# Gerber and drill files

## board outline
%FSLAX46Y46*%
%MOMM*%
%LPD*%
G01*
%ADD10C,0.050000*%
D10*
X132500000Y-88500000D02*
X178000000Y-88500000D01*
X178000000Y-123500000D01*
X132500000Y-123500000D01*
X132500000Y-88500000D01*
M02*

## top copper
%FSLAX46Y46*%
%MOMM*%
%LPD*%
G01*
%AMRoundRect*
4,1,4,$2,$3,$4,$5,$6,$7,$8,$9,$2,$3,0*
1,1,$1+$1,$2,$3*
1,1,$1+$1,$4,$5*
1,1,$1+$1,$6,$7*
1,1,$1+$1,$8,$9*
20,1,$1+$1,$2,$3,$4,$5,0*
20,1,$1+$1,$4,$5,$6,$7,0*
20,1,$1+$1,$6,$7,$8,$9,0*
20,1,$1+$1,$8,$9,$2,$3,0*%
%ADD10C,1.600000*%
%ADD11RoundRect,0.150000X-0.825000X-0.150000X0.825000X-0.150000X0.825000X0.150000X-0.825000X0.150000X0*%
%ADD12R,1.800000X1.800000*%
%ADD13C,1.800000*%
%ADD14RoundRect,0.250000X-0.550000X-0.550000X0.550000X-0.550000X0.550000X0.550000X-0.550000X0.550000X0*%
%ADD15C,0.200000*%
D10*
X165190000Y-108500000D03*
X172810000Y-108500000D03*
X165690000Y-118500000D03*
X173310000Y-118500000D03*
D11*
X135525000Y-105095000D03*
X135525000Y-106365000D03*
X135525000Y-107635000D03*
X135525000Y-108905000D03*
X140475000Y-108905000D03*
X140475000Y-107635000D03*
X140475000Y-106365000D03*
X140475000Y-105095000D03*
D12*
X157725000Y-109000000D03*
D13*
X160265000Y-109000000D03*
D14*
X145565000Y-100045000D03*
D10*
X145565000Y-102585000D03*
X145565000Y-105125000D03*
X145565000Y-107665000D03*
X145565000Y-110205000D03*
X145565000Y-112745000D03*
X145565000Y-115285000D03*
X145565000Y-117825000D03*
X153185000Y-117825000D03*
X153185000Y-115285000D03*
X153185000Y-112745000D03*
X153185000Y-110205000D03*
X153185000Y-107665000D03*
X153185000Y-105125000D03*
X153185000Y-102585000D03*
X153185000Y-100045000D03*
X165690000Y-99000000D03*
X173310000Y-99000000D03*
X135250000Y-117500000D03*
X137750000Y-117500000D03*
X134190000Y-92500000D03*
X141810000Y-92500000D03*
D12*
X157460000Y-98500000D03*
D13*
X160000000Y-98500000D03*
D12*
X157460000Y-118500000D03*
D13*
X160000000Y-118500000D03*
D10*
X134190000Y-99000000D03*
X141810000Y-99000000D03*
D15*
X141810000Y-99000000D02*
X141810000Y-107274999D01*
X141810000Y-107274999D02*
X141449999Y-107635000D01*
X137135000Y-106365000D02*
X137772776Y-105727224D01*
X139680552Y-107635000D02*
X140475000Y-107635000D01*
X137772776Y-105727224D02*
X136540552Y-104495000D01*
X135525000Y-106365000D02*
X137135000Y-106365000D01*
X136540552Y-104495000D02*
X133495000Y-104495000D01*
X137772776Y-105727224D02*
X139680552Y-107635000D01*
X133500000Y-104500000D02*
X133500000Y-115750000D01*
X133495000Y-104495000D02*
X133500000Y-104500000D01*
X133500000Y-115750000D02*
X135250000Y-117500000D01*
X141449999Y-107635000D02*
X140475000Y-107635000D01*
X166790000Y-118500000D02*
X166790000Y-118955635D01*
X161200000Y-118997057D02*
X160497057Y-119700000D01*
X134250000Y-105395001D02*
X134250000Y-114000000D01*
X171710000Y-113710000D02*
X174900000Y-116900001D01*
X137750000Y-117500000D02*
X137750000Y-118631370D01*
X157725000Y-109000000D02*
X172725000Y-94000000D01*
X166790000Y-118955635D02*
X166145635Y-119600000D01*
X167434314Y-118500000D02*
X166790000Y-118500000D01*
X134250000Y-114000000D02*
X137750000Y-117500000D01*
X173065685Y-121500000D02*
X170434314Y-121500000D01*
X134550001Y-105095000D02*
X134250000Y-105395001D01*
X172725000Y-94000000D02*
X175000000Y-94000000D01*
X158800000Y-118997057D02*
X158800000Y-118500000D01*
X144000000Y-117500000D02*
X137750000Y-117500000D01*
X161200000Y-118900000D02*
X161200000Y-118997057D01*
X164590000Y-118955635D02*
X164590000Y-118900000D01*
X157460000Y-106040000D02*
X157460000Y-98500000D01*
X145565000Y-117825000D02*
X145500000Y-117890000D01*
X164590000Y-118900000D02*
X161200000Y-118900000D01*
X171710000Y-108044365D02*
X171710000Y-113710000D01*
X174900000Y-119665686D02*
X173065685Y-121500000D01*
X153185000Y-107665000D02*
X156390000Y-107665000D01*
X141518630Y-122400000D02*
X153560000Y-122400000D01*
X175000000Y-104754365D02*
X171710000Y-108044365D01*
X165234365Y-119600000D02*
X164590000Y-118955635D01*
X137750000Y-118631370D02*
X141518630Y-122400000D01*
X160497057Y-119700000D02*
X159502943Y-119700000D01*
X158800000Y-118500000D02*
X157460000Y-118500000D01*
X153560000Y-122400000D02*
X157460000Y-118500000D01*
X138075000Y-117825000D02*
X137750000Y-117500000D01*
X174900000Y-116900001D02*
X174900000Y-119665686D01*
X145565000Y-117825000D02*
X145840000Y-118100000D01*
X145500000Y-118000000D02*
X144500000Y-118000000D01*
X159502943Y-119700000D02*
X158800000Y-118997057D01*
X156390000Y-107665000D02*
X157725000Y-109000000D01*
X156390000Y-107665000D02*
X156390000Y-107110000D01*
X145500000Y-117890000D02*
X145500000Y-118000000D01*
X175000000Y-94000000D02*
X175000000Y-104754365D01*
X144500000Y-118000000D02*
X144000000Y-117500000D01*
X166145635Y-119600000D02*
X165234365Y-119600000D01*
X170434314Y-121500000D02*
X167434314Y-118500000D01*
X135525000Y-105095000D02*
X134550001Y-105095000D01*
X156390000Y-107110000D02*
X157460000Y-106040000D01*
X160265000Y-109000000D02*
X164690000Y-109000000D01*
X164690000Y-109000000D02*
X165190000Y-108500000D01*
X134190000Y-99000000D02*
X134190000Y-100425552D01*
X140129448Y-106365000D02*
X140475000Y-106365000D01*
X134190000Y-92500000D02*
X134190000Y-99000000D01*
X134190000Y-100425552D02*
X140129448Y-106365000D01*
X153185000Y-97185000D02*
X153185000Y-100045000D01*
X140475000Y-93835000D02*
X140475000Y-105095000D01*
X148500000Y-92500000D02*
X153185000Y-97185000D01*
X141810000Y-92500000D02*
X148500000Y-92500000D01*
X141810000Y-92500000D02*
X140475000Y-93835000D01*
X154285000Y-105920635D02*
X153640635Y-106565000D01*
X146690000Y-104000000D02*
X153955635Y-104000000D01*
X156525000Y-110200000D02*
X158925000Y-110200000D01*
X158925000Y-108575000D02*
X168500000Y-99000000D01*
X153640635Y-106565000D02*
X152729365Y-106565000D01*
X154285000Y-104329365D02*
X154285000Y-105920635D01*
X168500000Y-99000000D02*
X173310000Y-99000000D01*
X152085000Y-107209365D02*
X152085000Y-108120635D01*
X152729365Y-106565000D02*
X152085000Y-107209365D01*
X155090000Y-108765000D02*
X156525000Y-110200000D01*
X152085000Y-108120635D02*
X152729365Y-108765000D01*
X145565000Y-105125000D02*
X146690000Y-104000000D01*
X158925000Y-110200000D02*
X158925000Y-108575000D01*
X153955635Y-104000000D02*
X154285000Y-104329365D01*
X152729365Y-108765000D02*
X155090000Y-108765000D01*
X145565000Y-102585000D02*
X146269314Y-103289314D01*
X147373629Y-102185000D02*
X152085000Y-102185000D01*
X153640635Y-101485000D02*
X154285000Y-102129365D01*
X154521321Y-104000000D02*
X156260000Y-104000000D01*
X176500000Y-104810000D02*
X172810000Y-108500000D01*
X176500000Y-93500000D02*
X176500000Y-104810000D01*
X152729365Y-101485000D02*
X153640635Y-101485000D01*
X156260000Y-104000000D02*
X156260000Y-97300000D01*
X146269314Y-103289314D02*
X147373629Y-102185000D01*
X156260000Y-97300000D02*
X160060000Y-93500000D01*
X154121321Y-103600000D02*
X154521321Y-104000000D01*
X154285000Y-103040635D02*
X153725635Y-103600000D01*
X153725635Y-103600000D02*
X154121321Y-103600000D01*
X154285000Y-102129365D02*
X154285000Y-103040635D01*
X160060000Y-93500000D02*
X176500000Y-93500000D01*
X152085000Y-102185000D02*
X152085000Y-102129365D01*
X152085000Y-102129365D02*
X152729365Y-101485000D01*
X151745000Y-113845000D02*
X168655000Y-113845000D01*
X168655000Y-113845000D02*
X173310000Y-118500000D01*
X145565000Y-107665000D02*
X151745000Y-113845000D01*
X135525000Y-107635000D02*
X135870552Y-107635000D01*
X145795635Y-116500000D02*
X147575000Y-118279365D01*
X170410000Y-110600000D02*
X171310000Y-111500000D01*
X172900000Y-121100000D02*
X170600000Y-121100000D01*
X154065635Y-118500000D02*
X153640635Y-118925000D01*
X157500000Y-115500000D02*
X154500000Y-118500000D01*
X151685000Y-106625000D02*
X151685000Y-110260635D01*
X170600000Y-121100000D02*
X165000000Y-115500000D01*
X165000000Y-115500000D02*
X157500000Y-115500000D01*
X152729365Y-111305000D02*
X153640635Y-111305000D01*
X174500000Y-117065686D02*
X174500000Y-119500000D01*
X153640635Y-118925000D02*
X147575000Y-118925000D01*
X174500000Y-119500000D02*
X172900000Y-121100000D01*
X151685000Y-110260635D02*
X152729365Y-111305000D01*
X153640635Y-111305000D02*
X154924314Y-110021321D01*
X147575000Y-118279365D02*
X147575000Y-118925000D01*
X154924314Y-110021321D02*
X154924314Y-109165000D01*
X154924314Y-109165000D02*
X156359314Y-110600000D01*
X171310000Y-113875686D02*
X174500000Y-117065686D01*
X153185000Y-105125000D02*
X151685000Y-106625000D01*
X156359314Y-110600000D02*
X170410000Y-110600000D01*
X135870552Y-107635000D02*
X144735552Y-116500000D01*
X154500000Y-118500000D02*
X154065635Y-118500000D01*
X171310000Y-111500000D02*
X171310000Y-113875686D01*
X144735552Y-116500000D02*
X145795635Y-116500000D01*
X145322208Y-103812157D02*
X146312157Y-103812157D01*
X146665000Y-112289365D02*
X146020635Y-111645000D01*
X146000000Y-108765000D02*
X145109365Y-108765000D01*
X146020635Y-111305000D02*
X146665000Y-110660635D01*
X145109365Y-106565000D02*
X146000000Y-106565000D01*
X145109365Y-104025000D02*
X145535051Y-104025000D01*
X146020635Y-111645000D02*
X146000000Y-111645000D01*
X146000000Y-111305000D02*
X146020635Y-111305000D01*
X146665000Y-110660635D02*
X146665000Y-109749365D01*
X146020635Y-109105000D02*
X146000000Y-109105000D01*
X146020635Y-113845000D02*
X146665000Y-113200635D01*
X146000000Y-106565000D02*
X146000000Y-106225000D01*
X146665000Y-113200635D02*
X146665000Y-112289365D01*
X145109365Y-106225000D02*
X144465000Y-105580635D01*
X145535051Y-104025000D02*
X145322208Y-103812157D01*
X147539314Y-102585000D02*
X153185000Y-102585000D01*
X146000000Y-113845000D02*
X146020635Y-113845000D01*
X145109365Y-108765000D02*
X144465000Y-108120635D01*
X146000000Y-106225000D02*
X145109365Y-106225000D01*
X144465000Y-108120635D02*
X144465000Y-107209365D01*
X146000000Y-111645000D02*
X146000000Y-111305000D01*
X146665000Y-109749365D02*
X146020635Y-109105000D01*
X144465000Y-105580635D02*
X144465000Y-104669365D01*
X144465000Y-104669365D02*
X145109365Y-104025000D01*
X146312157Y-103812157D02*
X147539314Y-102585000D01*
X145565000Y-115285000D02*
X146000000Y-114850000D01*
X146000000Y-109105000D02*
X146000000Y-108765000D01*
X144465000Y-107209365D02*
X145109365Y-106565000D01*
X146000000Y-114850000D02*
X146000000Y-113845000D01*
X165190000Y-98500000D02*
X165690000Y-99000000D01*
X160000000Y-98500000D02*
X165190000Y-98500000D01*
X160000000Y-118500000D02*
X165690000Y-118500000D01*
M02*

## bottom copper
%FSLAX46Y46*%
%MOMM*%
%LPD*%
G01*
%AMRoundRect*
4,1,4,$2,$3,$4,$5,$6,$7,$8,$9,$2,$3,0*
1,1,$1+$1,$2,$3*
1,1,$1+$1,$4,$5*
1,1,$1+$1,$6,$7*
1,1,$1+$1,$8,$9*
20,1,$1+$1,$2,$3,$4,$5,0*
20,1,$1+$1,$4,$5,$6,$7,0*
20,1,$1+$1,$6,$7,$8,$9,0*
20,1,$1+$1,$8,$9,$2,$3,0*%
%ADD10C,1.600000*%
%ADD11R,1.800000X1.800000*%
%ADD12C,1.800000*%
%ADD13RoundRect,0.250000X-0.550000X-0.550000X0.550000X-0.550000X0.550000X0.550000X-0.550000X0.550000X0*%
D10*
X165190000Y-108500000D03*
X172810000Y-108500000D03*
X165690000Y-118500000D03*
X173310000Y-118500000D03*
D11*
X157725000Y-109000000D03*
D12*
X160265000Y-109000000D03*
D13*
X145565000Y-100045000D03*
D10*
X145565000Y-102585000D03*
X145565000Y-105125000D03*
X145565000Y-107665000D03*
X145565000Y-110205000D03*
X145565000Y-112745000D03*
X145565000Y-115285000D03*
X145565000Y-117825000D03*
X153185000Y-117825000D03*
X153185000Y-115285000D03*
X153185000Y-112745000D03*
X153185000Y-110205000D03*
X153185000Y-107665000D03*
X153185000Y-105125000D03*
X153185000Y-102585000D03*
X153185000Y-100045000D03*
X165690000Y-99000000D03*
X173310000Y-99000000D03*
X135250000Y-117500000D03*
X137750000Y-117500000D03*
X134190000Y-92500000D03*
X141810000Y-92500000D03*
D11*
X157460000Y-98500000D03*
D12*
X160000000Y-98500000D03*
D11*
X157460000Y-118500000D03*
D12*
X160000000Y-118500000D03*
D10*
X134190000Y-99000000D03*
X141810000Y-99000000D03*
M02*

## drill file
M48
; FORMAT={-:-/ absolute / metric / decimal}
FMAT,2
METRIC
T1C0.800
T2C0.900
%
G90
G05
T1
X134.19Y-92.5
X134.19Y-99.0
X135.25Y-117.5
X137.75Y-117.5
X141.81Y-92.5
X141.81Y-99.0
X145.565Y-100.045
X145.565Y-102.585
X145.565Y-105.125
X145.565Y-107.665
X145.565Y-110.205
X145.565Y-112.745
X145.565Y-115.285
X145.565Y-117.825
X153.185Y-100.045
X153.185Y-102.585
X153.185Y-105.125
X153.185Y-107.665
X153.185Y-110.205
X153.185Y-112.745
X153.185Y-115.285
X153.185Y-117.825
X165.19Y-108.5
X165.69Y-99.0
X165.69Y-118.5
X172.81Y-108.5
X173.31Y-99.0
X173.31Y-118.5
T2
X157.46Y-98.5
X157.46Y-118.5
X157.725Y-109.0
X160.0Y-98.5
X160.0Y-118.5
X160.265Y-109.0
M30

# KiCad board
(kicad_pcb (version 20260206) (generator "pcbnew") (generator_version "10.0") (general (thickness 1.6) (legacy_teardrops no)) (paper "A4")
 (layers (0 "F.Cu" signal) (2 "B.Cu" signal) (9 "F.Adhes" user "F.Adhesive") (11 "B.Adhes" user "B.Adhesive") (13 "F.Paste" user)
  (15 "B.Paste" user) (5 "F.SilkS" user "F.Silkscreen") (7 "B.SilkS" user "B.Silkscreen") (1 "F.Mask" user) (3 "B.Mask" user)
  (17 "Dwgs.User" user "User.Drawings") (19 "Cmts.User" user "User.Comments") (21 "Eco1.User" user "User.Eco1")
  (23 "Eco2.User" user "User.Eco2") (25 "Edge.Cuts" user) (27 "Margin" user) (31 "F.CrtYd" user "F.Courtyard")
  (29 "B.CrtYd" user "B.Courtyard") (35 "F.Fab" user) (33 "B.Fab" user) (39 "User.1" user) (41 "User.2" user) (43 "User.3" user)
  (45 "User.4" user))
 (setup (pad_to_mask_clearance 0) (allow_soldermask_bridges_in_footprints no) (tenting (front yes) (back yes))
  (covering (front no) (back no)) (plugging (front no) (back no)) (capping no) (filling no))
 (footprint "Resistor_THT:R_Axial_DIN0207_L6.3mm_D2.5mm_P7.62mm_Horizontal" (layer "F.Cu") (at 165.19 108.5)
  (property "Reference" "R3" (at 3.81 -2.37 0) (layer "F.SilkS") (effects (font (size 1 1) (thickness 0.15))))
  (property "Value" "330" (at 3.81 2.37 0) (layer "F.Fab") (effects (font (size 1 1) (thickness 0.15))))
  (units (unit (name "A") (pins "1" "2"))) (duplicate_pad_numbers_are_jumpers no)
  (pad "1" thru_hole circle (at 0 0) (size 1.6 1.6) (drill 0.8) (layers "*.Cu" "*.Mask") (remove_unused_layers no) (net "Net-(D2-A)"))
  (pad "2" thru_hole circle (at 7.62 0) (size 1.6 1.6) (drill 0.8) (layers "*.Cu" "*.Mask") (remove_unused_layers no) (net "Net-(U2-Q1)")))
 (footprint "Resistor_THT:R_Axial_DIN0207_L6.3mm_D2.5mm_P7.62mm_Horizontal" (layer "F.Cu") (at 165.69 118.5)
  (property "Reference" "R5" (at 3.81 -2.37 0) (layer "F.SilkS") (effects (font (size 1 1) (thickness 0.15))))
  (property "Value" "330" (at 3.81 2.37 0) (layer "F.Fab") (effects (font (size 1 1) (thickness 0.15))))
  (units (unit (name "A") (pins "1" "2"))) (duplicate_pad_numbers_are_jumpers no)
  (pad "1" thru_hole circle (at 0 0) (size 1.6 1.6) (drill 0.8) (layers "*.Cu" "*.Mask") (remove_unused_layers no) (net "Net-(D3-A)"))
  (pad "2" thru_hole circle (at 7.62 0) (size 1.6 1.6) (drill 0.8) (layers "*.Cu" "*.Mask") (remove_unused_layers no) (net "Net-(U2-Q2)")))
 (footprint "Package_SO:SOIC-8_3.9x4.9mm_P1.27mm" (layer "F.Cu") (at 138 107)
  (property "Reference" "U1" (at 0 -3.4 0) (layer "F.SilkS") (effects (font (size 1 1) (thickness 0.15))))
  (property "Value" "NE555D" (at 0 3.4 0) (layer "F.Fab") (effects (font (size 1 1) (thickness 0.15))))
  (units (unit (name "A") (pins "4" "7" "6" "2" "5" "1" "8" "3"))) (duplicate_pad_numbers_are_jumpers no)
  (pad "1" smd roundrect (at -2.475 -1.905) (size 1.95 0.6) (layers "F.Cu" "F.Mask" "F.Paste") (roundrect_rratio 0.25) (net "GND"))
  (pad "2" smd roundrect (at -2.475 -0.635) (size 1.95 0.6) (layers "F.Cu" "F.Mask" "F.Paste") (roundrect_rratio 0.25)
   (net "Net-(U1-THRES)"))
  (pad "3" smd roundrect (at -2.475 0.635) (size 1.95 0.6) (layers "F.Cu" "F.Mask" "F.Paste") (roundrect_rratio 0.25) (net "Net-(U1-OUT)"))
  (pad "4" smd roundrect (at -2.475 1.905) (size 1.95 0.6) (layers "F.Cu" "F.Mask" "F.Paste") (roundrect_rratio 0.25)
   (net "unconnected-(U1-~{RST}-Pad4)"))
  (pad "5" smd roundrect (at 2.475 1.905) (size 1.95 0.6) (layers "F.Cu" "F.Mask" "F.Paste") (roundrect_rratio 0.25)
   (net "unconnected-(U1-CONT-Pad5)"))
  (pad "6" smd roundrect (at 2.475 0.635) (size 1.95 0.6) (layers "F.Cu" "F.Mask" "F.Paste") (roundrect_rratio 0.25) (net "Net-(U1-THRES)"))
  (pad "7" smd roundrect (at 2.475 -0.635) (size 1.95 0.6) (layers "F.Cu" "F.Mask" "F.Paste") (roundrect_rratio 0.25) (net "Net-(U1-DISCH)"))
  (pad "8" smd roundrect (at 2.475 -1.905) (size 1.95 0.6) (layers "F.Cu" "F.Mask" "F.Paste") (roundrect_rratio 0.25) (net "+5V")))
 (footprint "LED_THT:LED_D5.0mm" (layer "F.Cu") (at 157.725 109)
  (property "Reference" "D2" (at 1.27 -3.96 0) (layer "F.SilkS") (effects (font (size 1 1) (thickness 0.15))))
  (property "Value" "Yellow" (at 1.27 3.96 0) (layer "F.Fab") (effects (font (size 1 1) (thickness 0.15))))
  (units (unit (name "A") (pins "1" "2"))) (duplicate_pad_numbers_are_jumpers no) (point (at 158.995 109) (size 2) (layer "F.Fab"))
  (pad "1" thru_hole rect (at 0 0) (size 1.8 1.8) (drill 0.9) (layers "*.Cu" "*.Mask") (remove_unused_layers no) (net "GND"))
  (pad "2" thru_hole circle (at 2.54 0) (size 1.8 1.8) (drill 0.9) (layers "*.Cu" "*.Mask") (remove_unused_layers no) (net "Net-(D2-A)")))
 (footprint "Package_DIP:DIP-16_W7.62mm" (layer "F.Cu") (at 145.565 100.045)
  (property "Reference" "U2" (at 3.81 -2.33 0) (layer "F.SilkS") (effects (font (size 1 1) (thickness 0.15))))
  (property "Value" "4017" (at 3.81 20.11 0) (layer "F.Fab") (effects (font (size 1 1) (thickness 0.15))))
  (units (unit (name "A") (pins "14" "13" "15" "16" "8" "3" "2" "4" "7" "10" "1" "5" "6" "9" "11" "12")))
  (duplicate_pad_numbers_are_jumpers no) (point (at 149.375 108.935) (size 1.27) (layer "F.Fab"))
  (pad "1" thru_hole roundrect (at 0 0) (size 1.6 1.6) (drill 0.8) (layers "*.Cu" "*.Mask") (remove_unused_layers no)
   (roundrect_rratio 0.15625) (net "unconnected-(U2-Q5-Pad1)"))
  (pad "2" thru_hole circle (at 0 2.54) (size 1.6 1.6) (drill 0.8) (layers "*.Cu" "*.Mask") (remove_unused_layers no) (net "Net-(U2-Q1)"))
  (pad "3" thru_hole circle (at 0 5.08) (size 1.6 1.6) (drill 0.8) (layers "*.Cu" "*.Mask") (remove_unused_layers no) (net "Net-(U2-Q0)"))
  (pad "4" thru_hole circle (at 0 7.62) (size 1.6 1.6) (drill 0.8) (layers "*.Cu" "*.Mask") (remove_unused_layers no) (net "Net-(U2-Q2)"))
  (pad "5" thru_hole circle (at 0 10.16) (size 1.6 1.6) (drill 0.8) (layers "*.Cu" "*.Mask") (remove_unused_layers no)
   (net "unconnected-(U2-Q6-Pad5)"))
  (pad "6" thru_hole circle (at 0 12.7) (size 1.6 1.6) (drill 0.8) (layers "*.Cu" "*.Mask") (remove_unused_layers no)
   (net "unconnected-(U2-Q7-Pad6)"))
  (pad "7" thru_hole circle (at 0 15.24) (size 1.6 1.6) (drill 0.8) (layers "*.Cu" "*.Mask") (remove_unused_layers no) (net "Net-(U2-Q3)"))
  (pad "8" thru_hole circle (at 0 17.78) (size 1.6 1.6) (drill 0.8) (layers "*.Cu" "*.Mask") (remove_unused_layers no) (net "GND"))
  (pad "9" thru_hole circle (at 7.62 17.78) (size 1.6 1.6) (drill 0.8) (layers "*.Cu" "*.Mask") (remove_unused_layers no)
   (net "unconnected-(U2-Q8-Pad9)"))
  (pad "10" thru_hole circle (at 7.62 15.24) (size 1.6 1.6) (drill 0.8) (layers "*.Cu" "*.Mask") (remove_unused_layers no)
   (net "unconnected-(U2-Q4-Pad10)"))
  (pad "11" thru_hole circle (at 7.62 12.7) (size 1.6 1.6) (drill 0.8) (layers "*.Cu" "*.Mask") (remove_unused_layers no)
   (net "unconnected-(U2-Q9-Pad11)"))
  (pad "12" thru_hole circle (at 7.62 10.16) (size 1.6 1.6) (drill 0.8) (layers "*.Cu" "*.Mask") (remove_unused_layers no)
   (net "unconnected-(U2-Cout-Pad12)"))
  (pad "13" thru_hole circle (at 7.62 7.62) (size 1.6 1.6) (drill 0.8) (layers "*.Cu" "*.Mask") (remove_unused_layers no) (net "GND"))
  (pad "14" thru_hole circle (at 7.62 5.08) (size 1.6 1.6) (drill 0.8) (layers "*.Cu" "*.Mask") (remove_unused_layers no)
   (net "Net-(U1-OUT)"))
  (pad "15" thru_hole circle (at 7.62 2.54) (size 1.6 1.6) (drill 0.8) (layers "*.Cu" "*.Mask") (remove_unused_layers no)
   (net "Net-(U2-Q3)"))
  (pad "16" thru_hole circle (at 7.62 0) (size 1.6 1.6) (drill 0.8) (layers "*.Cu" "*.Mask") (remove_unused_layers no) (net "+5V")))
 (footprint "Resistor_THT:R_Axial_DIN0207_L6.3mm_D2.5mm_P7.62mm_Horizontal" (layer "F.Cu") (at 165.69 99)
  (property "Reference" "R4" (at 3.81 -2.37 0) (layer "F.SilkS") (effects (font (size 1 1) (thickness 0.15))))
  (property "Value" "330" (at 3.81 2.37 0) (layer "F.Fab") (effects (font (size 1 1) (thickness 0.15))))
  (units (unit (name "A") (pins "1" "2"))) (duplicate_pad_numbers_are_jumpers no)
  (pad "1" thru_hole circle (at 0 0) (size 1.6 1.6) (drill 0.8) (layers "*.Cu" "*.Mask") (remove_unused_layers no) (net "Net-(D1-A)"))
  (pad "2" thru_hole circle (at 7.62 0) (size 1.6 1.6) (drill 0.8) (layers "*.Cu" "*.Mask") (remove_unused_layers no) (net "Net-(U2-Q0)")))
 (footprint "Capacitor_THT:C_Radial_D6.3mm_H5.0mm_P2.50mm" (layer "F.Cu") (at 135.25 117.5)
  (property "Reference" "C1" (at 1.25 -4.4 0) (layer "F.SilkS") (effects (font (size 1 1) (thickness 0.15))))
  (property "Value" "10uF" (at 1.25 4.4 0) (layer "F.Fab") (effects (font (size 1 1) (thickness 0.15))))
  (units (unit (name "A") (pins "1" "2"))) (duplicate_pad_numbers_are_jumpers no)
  (pad "1" thru_hole circle (at 0 0) (size 1.6 1.6) (drill 0.8) (layers "*.Cu" "*.Mask") (remove_unused_layers no) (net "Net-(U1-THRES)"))
  (pad "2" thru_hole circle (at 2.5 0) (size 1.6 1.6) (drill 0.8) (layers "*.Cu" "*.Mask") (remove_unused_layers no) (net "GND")))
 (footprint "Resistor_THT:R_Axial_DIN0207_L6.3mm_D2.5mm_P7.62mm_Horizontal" (layer "F.Cu") (at 134.19 92.5)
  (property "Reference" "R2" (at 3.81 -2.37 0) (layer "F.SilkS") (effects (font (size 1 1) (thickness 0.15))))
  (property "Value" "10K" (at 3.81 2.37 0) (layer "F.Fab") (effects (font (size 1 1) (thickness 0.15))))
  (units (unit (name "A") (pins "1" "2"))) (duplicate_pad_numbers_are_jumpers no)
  (pad "1" thru_hole circle (at 0 0) (size 1.6 1.6) (drill 0.8) (layers "*.Cu" "*.Mask") (remove_unused_layers no) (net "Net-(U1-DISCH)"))
  (pad "2" thru_hole circle (at 7.62 0) (size 1.6 1.6) (drill 0.8) (layers "*.Cu" "*.Mask") (remove_unused_layers no) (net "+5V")))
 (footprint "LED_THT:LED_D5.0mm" (layer "F.Cu") (at 157.46 98.5)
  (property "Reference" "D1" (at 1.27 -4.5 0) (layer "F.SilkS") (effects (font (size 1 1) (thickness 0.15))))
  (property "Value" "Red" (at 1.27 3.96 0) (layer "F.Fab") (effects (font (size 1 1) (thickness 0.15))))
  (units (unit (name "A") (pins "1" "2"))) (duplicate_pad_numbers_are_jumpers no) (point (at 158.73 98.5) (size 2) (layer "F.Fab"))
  (pad "1" thru_hole rect (at 0 0) (size 1.8 1.8) (drill 0.9) (layers "*.Cu" "*.Mask") (remove_unused_layers no) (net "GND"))
  (pad "2" thru_hole circle (at 2.54 0) (size 1.8 1.8) (drill 0.9) (layers "*.Cu" "*.Mask") (remove_unused_layers no) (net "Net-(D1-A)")))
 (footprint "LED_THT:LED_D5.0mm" (layer "F.Cu") (at 157.46 118.5)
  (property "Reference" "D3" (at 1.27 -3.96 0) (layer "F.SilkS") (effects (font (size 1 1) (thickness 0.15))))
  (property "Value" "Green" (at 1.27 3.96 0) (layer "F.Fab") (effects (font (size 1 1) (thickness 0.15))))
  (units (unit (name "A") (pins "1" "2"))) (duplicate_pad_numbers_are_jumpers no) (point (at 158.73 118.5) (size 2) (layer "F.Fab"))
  (pad "1" thru_hole rect (at 0 0) (size 1.8 1.8) (drill 0.9) (layers "*.Cu" "*.Mask") (remove_unused_layers no) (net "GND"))
  (pad "2" thru_hole circle (at 2.54 0) (size 1.8 1.8) (drill 0.9) (layers "*.Cu" "*.Mask") (remove_unused_layers no)))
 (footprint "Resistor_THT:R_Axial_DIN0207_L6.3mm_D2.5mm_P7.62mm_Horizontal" (layer "F.Cu") (at 134.19 99)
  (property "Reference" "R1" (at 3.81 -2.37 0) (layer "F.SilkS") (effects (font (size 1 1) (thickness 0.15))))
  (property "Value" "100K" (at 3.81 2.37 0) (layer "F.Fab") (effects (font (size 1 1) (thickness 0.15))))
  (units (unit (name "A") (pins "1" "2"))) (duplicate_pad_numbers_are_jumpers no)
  (pad "1" thru_hole circle (at 0 0) (size 1.6 1.6) (drill 0.8) (layers "*.Cu" "*.Mask") (remove_unused_layers no) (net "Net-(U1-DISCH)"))
  (pad "2" thru_hole circle (at 7.62 0) (size 1.6 1.6) (drill 0.8) (layers "*.Cu" "*.Mask") (remove_unused_layers no) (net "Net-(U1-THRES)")))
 (gr_rect (start 132.5 88.5) (end 178 123.5) (stroke (width 0.05) (type default)) (fill no) (layer "Edge.Cuts"))
 (segment (start 141.81 99) (end 141.81 107.274999) (width 0.2) (layer "F.Cu") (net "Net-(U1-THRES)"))
 (segment (start 141.81 107.274999) (end 141.449999 107.635) (width 0.2) (layer "F.Cu") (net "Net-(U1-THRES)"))
 (segment (start 137.135 106.365) (end 137.772776 105.727224) (width 0.2) (layer "F.Cu") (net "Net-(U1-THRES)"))
 (segment (start 139.680552 107.635) (end 140.475 107.635) (width 0.2) (layer "F.Cu") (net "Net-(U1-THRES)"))
 (segment (start 137.772776 105.727224) (end 136.540552 104.495) (width 0.2) (layer "F.Cu") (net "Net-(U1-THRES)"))
 (segment (start 135.525 106.365) (end 137.135 106.365) (width 0.2) (layer "F.Cu") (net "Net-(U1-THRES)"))
 (segment (start 136.540552 104.495) (end 133.495 104.495) (width 0.2) (layer "F.Cu") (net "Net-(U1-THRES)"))
 (segment (start 137.772776 105.727224) (end 139.680552 107.635) (width 0.2) (layer "F.Cu") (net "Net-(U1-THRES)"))
 (segment (start 133.5 104.5) (end 133.5 115.75) (width 0.2) (layer "F.Cu") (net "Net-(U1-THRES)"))
 (segment (start 133.495 104.495) (end 133.5 104.5) (width 0.2) (layer "F.Cu") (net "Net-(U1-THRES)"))
 (segment (start 133.5 115.75) (end 135.25 117.5) (width 0.2) (layer "F.Cu") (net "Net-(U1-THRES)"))
 (segment (start 141.449999 107.635) (end 140.475 107.635) (width 0.2) (layer "F.Cu") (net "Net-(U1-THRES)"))
 (segment (start 166.79 118.5) (end 166.79 118.955635) (width 0.2) (layer "F.Cu") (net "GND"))
 (segment (start 161.2 118.997057) (end 160.497057 119.7) (width 0.2) (layer "F.Cu") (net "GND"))
 (segment (start 134.25 105.395001) (end 134.25 114) (width 0.2) (layer "F.Cu") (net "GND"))
 (segment (start 171.71 113.71) (end 174.9 116.900001) (width 0.2) (layer "F.Cu") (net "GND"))
 (segment (start 137.75 117.5) (end 137.75 118.63137) (width 0.2) (layer "F.Cu") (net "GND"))
 (segment (start 157.725 109) (end 172.725 94) (width 0.2) (layer "F.Cu") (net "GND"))
 (segment (start 166.79 118.955635) (end 166.145635 119.6) (width 0.2) (layer "F.Cu") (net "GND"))
 (segment (start 167.434314 118.5) (end 166.79 118.5) (width 0.2) (layer "F.Cu") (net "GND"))
 (segment (start 134.25 114) (end 137.75 117.5) (width 0.2) (layer "F.Cu") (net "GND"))
 (segment (start 173.065685 121.5) (end 170.434314 121.5) (width 0.2) (layer "F.Cu") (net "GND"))
 (segment (start 134.550001 105.095) (end 134.25 105.395001) (width 0.2) (layer "F.Cu") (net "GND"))
 (segment (start 172.725 94) (end 175 94) (width 0.2) (layer "F.Cu") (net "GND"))
 (segment (start 158.8 118.997057) (end 158.8 118.5) (width 0.2) (layer "F.Cu") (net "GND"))
 (segment (start 144 117.5) (end 137.75 117.5) (width 0.2) (layer "F.Cu") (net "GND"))
 (segment (start 161.2 118.9) (end 161.2 118.997057) (width 0.2) (layer "F.Cu") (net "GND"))
 (segment (start 164.59 118.955635) (end 164.59 118.9) (width 0.2) (layer "F.Cu") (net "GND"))
 (segment (start 157.46 106.04) (end 157.46 98.5) (width 0.2) (layer "F.Cu") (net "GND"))
 (segment (start 145.565 117.825) (end 145.5 117.89) (width 0.2) (layer "F.Cu") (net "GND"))
 (segment (start 164.59 118.9) (end 161.2 118.9) (width 0.2) (layer "F.Cu") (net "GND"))
 (segment (start 171.71 108.044365) (end 171.71 113.71) (width 0.2) (layer "F.Cu") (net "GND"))
 (segment (start 174.9 119.665686) (end 173.065685 121.5) (width 0.2) (layer "F.Cu") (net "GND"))
 (segment (start 153.185 107.665) (end 156.39 107.665) (width 0.2) (layer "F.Cu") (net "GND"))
 (segment (start 141.51863 122.4) (end 153.56 122.4) (width 0.2) (layer "F.Cu") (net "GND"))
 (segment (start 175 104.754365) (end 171.71 108.044365) (width 0.2) (layer "F.Cu") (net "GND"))
 (segment (start 165.234365 119.6) (end 164.59 118.955635) (width 0.2) (layer "F.Cu") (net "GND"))
 (segment (start 137.75 118.63137) (end 141.51863 122.4) (width 0.2) (layer "F.Cu") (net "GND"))
 (segment (start 160.497057 119.7) (end 159.502943 119.7) (width 0.2) (layer "F.Cu") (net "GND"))
 (segment (start 158.8 118.5) (end 157.46 118.5) (width 0.2) (layer "F.Cu") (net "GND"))
 (segment (start 153.56 122.4) (end 157.46 118.5) (width 0.2) (layer "F.Cu") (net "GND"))
 (segment (start 138.075 117.825) (end 137.75 117.5) (width 0.2) (layer "F.Cu") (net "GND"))
 (segment (start 174.9 116.900001) (end 174.9 119.665686) (width 0.2) (layer "F.Cu") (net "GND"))
 (segment (start 145.565 117.825) (end 145.84 118.1) (width 0.2) (layer "F.Cu") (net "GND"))
 (segment (start 145.5 118) (end 144.5 118) (width 0.2) (layer "F.Cu") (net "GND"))
 (segment (start 159.502943 119.7) (end 158.8 118.997057) (width 0.2) (layer "F.Cu") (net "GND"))
 (segment (start 156.39 107.665) (end 157.725 109) (width 0.2) (layer "F.Cu") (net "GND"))
 (segment (start 156.39 107.665) (end 156.39 107.11) (width 0.2) (layer "F.Cu") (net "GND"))
 (segment (start 145.5 117.89) (end 145.5 118) (width 0.2) (layer "F.Cu") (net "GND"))
 (segment (start 175 94) (end 175 104.754365) (width 0.2) (layer "F.Cu") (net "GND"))
 (segment (start 144.5 118) (end 144 117.5) (width 0.2) (layer "F.Cu") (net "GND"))
 (segment (start 166.145635 119.6) (end 165.234365 119.6) (width 0.2) (layer "F.Cu") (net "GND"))
 (segment (start 170.434314 121.5) (end 167.434314 118.5) (width 0.2) (layer "F.Cu") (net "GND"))
 (segment (start 135.525 105.095) (end 134.550001 105.095) (width 0.2) (layer "F.Cu") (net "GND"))
 (segment (start 156.39 107.11) (end 157.46 106.04) (width 0.2) (layer "F.Cu") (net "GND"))
 (segment (start 160.265 109) (end 164.69 109) (width 0.2) (layer "F.Cu") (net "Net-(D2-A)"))
 (segment (start 164.69 109) (end 165.19 108.5) (width 0.2) (layer "F.Cu") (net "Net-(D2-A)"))
 (segment (start 134.19 99) (end 134.19 100.425552) (width 0.2) (layer "F.Cu") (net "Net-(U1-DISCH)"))
 (segment (start 140.129448 106.365) (end 140.475 106.365) (width 0.2) (layer "F.Cu") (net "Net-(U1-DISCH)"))
 (segment (start 134.19 92.5) (end 134.19 99) (width 0.2) (layer "F.Cu") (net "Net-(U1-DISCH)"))
 (segment (start 134.19 100.425552) (end 140.129448 106.365) (width 0.2) (layer "F.Cu") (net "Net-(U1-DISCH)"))
 (segment (start 153.185 97.185) (end 153.185 100.045) (width 0.2) (layer "F.Cu") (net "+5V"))
 (segment (start 140.475 93.835) (end 140.475 105.095) (width 0.2) (layer "F.Cu") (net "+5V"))
 (segment (start 148.5 92.5) (end 153.185 97.185) (width 0.2) (layer "F.Cu") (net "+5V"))
 (segment (start 141.81 92.5) (end 148.5 92.5) (width 0.2) (layer "F.Cu") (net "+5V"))
 (segment (start 141.81 92.5) (end 140.475 93.835) (width 0.2) (layer "F.Cu") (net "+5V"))
 (segment (start 154.285 105.920635) (end 153.640635 106.565) (width 0.2) (layer "F.Cu") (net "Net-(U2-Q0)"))
 (segment (start 146.69 104) (end 153.955635 104) (width 0.2) (layer "F.Cu") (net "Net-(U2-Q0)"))
 (segment (start 156.525 110.2) (end 158.925 110.2) (width 0.2) (layer "F.Cu") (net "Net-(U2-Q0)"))
 (segment (start 158.925 108.575) (end 168.5 99) (width 0.2) (layer "F.Cu") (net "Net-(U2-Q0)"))
 (segment (start 153.640635 106.565) (end 152.729365 106.565) (width 0.2) (layer "F.Cu") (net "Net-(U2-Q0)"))
 (segment (start 154.285 104.329365) (end 154.285 105.920635) (width 0.2) (layer "F.Cu") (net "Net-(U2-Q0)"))
 (segment (start 168.5 99) (end 173.31 99) (width 0.2) (layer "F.Cu") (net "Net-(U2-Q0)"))
 (segment (start 152.085 107.209365) (end 152.085 108.120635) (width 0.2) (layer "F.Cu") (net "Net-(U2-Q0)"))
 (segment (start 152.729365 106.565) (end 152.085 107.209365) (width 0.2) (layer "F.Cu") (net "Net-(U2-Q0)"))
 (segment (start 155.09 108.765) (end 156.525 110.2) (width 0.2) (layer "F.Cu") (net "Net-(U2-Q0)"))
 (segment (start 152.085 108.120635) (end 152.729365 108.765) (width 0.2) (layer "F.Cu") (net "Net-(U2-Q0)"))
 (segment (start 145.565 105.125) (end 146.69 104) (width 0.2) (layer "F.Cu") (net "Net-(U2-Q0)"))
 (segment (start 158.925 110.2) (end 158.925 108.575) (width 0.2) (layer "F.Cu") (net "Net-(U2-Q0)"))
 (segment (start 153.955635 104) (end 154.285 104.329365) (width 0.2) (layer "F.Cu") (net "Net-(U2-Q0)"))
 (segment (start 152.729365 108.765) (end 155.09 108.765) (width 0.2) (layer "F.Cu") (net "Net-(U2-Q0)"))
 (segment (start 145.565 102.585) (end 146.269314 103.289314) (width 0.2) (layer "F.Cu") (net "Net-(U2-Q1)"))
 (segment (start 147.373629 102.185) (end 152.085 102.185) (width 0.2) (layer "F.Cu") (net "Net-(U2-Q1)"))
 (segment (start 153.640635 101.485) (end 154.285 102.129365) (width 0.2) (layer "F.Cu") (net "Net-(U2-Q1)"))
 (segment (start 154.521321 104) (end 156.26 104) (width 0.2) (layer "F.Cu") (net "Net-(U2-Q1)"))
 (segment (start 176.5 104.81) (end 172.81 108.5) (width 0.2) (layer "F.Cu") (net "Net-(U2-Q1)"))
 (segment (start 176.5 93.5) (end 176.5 104.81) (width 0.2) (layer "F.Cu") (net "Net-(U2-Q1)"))
 (segment (start 152.729365 101.485) (end 153.640635 101.485) (width 0.2) (layer "F.Cu") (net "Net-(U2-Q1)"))
 (segment (start 156.26 104) (end 156.26 97.3) (width 0.2) (layer "F.Cu") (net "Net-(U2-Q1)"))
 (segment (start 146.269314 103.289314) (end 147.373629 102.185) (width 0.2) (layer "F.Cu") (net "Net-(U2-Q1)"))
 (segment (start 156.26 97.3) (end 160.06 93.5) (width 0.2) (layer "F.Cu") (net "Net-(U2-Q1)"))
 (segment (start 154.121321 103.6) (end 154.521321 104) (width 0.2) (layer "F.Cu") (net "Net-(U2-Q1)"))
 (segment (start 154.285 103.040635) (end 153.725635 103.6) (width 0.2) (layer "F.Cu") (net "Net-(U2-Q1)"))
 (segment (start 153.725635 103.6) (end 154.121321 103.6) (width 0.2) (layer "F.Cu") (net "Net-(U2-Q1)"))
 (segment (start 154.285 102.129365) (end 154.285 103.040635) (width 0.2) (layer "F.Cu") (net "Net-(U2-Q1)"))
 (segment (start 160.06 93.5) (end 176.5 93.5) (width 0.2) (layer "F.Cu") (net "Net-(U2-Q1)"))
 (segment (start 152.085 102.185) (end 152.085 102.129365) (width 0.2) (layer "F.Cu") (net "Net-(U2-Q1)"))
 (segment (start 152.085 102.129365) (end 152.729365 101.485) (width 0.2) (layer "F.Cu") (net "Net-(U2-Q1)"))
 (segment (start 151.745 113.845) (end 168.655 113.845) (width 0.2) (layer "F.Cu") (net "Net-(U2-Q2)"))
 (segment (start 168.655 113.845) (end 173.31 118.5) (width 0.2) (layer "F.Cu") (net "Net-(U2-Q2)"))
 (segment (start 145.565 107.665) (end 151.745 113.845) (width 0.2) (layer "F.Cu") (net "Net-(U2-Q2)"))
 (segment (start 135.525 107.635) (end 135.870552 107.635) (width 0.2) (layer "F.Cu") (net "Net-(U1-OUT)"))
 (segment (start 145.795635 116.5) (end 147.575 118.279365) (width 0.2) (layer "F.Cu") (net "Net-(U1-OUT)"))
 (segment (start 170.41 110.6) (end 171.31 111.5) (width 0.2) (layer "F.Cu") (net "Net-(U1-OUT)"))
 (segment (start 172.9 121.1) (end 170.6 121.1) (width 0.2) (layer "F.Cu") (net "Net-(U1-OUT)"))
 (segment (start 154.065635 118.5) (end 153.640635 118.925) (width 0.2) (layer "F.Cu") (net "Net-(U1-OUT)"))
 (segment (start 157.5 115.5) (end 154.5 118.5) (width 0.2) (layer "F.Cu") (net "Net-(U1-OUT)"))
 (segment (start 151.685 106.625) (end 151.685 110.260635) (width 0.2) (layer "F.Cu") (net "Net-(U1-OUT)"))
 (segment (start 170.6 121.1) (end 165 115.5) (width 0.2) (layer "F.Cu") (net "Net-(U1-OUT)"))
 (segment (start 165 115.5) (end 157.5 115.5) (width 0.2) (layer "F.Cu") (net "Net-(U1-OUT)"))
 (segment (start 152.729365 111.305) (end 153.640635 111.305) (width 0.2) (layer "F.Cu") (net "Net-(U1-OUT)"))
 (segment (start 174.5 117.065686) (end 174.5 119.5) (width 0.2) (layer "F.Cu") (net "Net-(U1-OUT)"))
 (segment (start 153.640635 118.925) (end 147.575 118.925) (width 0.2) (layer "F.Cu") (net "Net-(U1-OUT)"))
 (segment (start 174.5 119.5) (end 172.9 121.1) (width 0.2) (layer "F.Cu") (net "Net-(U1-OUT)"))
 (segment (start 151.685 110.260635) (end 152.729365 111.305) (width 0.2) (layer "F.Cu") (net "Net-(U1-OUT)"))
 (segment (start 153.640635 111.305) (end 154.924314 110.021321) (width 0.2) (layer "F.Cu") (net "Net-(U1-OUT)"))
 (segment (start 147.575 118.279365) (end 147.575 118.925) (width 0.2) (layer "F.Cu") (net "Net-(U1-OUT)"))
 (segment (start 154.924314 110.021321) (end 154.924314 109.165) (width 0.2) (layer "F.Cu") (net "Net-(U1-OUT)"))
 (segment (start 154.924314 109.165) (end 156.359314 110.6) (width 0.2) (layer "F.Cu") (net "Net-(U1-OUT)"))
 (segment (start 171.31 113.875686) (end 174.5 117.065686) (width 0.2) (layer "F.Cu") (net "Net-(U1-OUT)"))
 (segment (start 153.185 105.125) (end 151.685 106.625) (width 0.2) (layer "F.Cu") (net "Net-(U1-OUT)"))
 (segment (start 156.359314 110.6) (end 170.41 110.6) (width 0.2) (layer "F.Cu") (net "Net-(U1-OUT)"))
 (segment (start 135.870552 107.635) (end 144.735552 116.5) (width 0.2) (layer "F.Cu") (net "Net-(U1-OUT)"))
 (segment (start 154.5 118.5) (end 154.065635 118.5) (width 0.2) (layer "F.Cu") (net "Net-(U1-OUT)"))
 (segment (start 171.31 111.5) (end 171.31 113.875686) (width 0.2) (layer "F.Cu") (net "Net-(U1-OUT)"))
 (segment (start 144.735552 116.5) (end 145.795635 116.5) (width 0.2) (layer "F.Cu") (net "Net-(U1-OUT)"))
 (segment (start 145.322208 103.812157) (end 146.312157 103.812157) (width 0.2) (layer "F.Cu") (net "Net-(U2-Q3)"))
 (segment (start 146.665 112.289365) (end 146.020635 111.645) (width 0.2) (layer "F.Cu") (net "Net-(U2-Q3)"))
 (segment (start 146 108.765) (end 145.109365 108.765) (width 0.2) (layer "F.Cu") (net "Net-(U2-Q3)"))
 (segment (start 146.020635 111.305) (end 146.665 110.660635) (width 0.2) (layer "F.Cu") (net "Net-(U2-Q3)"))
 (segment (start 145.109365 106.565) (end 146 106.565) (width 0.2) (layer "F.Cu") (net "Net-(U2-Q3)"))
 (segment (start 145.109365 104.025) (end 145.535051 104.025) (width 0.2) (layer "F.Cu") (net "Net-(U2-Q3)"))
 (segment (start 146.020635 111.645) (end 146 111.645) (width 0.2) (layer "F.Cu") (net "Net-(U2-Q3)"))
 (segment (start 146 111.305) (end 146.020635 111.305) (width 0.2) (layer "F.Cu") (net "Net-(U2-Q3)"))
 (segment (start 146.665 110.660635) (end 146.665 109.749365) (width 0.2) (layer "F.Cu") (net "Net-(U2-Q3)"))
 (segment (start 146.020635 109.105) (end 146 109.105) (width 0.2) (layer "F.Cu") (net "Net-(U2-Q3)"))
 (segment (start 146.020635 113.845) (end 146.665 113.200635) (width 0.2) (layer "F.Cu") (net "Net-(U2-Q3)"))
 (segment (start 146 106.565) (end 146 106.225) (width 0.2) (layer "F.Cu") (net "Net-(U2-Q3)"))
 (segment (start 146.665 113.200635) (end 146.665 112.289365) (width 0.2) (layer "F.Cu") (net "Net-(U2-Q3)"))
 (segment (start 145.109365 106.225) (end 144.465 105.580635) (width 0.2) (layer "F.Cu") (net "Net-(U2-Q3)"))
 (segment (start 145.535051 104.025) (end 145.322208 103.812157) (width 0.2) (layer "F.Cu") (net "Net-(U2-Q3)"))
 (segment (start 147.539314 102.585) (end 153.185 102.585) (width 0.2) (layer "F.Cu") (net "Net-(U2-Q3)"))
 (segment (start 146 113.845) (end 146.020635 113.845) (width 0.2) (layer "F.Cu") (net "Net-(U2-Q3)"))
 (segment (start 145.109365 108.765) (end 144.465 108.120635) (width 0.2) (layer "F.Cu") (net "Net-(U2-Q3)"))
 (segment (start 146 106.225) (end 145.109365 106.225) (width 0.2) (layer "F.Cu") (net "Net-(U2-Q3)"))
 (segment (start 144.465 108.120635) (end 144.465 107.209365) (width 0.2) (layer "F.Cu") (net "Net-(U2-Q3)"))
 (segment (start 146 111.645) (end 146 111.305) (width 0.2) (layer "F.Cu") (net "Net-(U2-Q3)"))
 (segment (start 146.665 109.749365) (end 146.020635 109.105) (width 0.2) (layer "F.Cu") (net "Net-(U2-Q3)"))
 (segment (start 144.465 105.580635) (end 144.465 104.669365) (width 0.2) (layer "F.Cu") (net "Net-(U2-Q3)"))
 (segment (start 144.465 104.669365) (end 145.109365 104.025) (width 0.2) (layer "F.Cu") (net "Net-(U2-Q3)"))
 (segment (start 146.312157 103.812157) (end 147.539314 102.585) (width 0.2) (layer "F.Cu") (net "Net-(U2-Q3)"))
 (segment (start 145.565 115.285) (end 146 114.85) (width 0.2) (layer "F.Cu") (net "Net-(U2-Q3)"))
 (segment (start 146 109.105) (end 146 108.765) (width 0.2) (layer "F.Cu") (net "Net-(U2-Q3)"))
 (segment (start 144.465 107.209365) (end 145.109365 106.565) (width 0.2) (layer "F.Cu") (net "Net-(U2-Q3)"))
 (segment (start 146 114.85) (end 146 113.845) (width 0.2) (layer "F.Cu") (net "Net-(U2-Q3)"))
 (segment (start 165.19 98.5) (end 165.69 99) (width 0.2) (layer "F.Cu") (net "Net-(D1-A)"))
 (segment (start 160 98.5) (end 165.19 98.5) (width 0.2) (layer "F.Cu") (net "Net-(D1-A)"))
 (segment (start 160 118.5) (end 165.69 118.5) (width 0.2) (layer "F.Cu") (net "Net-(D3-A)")))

